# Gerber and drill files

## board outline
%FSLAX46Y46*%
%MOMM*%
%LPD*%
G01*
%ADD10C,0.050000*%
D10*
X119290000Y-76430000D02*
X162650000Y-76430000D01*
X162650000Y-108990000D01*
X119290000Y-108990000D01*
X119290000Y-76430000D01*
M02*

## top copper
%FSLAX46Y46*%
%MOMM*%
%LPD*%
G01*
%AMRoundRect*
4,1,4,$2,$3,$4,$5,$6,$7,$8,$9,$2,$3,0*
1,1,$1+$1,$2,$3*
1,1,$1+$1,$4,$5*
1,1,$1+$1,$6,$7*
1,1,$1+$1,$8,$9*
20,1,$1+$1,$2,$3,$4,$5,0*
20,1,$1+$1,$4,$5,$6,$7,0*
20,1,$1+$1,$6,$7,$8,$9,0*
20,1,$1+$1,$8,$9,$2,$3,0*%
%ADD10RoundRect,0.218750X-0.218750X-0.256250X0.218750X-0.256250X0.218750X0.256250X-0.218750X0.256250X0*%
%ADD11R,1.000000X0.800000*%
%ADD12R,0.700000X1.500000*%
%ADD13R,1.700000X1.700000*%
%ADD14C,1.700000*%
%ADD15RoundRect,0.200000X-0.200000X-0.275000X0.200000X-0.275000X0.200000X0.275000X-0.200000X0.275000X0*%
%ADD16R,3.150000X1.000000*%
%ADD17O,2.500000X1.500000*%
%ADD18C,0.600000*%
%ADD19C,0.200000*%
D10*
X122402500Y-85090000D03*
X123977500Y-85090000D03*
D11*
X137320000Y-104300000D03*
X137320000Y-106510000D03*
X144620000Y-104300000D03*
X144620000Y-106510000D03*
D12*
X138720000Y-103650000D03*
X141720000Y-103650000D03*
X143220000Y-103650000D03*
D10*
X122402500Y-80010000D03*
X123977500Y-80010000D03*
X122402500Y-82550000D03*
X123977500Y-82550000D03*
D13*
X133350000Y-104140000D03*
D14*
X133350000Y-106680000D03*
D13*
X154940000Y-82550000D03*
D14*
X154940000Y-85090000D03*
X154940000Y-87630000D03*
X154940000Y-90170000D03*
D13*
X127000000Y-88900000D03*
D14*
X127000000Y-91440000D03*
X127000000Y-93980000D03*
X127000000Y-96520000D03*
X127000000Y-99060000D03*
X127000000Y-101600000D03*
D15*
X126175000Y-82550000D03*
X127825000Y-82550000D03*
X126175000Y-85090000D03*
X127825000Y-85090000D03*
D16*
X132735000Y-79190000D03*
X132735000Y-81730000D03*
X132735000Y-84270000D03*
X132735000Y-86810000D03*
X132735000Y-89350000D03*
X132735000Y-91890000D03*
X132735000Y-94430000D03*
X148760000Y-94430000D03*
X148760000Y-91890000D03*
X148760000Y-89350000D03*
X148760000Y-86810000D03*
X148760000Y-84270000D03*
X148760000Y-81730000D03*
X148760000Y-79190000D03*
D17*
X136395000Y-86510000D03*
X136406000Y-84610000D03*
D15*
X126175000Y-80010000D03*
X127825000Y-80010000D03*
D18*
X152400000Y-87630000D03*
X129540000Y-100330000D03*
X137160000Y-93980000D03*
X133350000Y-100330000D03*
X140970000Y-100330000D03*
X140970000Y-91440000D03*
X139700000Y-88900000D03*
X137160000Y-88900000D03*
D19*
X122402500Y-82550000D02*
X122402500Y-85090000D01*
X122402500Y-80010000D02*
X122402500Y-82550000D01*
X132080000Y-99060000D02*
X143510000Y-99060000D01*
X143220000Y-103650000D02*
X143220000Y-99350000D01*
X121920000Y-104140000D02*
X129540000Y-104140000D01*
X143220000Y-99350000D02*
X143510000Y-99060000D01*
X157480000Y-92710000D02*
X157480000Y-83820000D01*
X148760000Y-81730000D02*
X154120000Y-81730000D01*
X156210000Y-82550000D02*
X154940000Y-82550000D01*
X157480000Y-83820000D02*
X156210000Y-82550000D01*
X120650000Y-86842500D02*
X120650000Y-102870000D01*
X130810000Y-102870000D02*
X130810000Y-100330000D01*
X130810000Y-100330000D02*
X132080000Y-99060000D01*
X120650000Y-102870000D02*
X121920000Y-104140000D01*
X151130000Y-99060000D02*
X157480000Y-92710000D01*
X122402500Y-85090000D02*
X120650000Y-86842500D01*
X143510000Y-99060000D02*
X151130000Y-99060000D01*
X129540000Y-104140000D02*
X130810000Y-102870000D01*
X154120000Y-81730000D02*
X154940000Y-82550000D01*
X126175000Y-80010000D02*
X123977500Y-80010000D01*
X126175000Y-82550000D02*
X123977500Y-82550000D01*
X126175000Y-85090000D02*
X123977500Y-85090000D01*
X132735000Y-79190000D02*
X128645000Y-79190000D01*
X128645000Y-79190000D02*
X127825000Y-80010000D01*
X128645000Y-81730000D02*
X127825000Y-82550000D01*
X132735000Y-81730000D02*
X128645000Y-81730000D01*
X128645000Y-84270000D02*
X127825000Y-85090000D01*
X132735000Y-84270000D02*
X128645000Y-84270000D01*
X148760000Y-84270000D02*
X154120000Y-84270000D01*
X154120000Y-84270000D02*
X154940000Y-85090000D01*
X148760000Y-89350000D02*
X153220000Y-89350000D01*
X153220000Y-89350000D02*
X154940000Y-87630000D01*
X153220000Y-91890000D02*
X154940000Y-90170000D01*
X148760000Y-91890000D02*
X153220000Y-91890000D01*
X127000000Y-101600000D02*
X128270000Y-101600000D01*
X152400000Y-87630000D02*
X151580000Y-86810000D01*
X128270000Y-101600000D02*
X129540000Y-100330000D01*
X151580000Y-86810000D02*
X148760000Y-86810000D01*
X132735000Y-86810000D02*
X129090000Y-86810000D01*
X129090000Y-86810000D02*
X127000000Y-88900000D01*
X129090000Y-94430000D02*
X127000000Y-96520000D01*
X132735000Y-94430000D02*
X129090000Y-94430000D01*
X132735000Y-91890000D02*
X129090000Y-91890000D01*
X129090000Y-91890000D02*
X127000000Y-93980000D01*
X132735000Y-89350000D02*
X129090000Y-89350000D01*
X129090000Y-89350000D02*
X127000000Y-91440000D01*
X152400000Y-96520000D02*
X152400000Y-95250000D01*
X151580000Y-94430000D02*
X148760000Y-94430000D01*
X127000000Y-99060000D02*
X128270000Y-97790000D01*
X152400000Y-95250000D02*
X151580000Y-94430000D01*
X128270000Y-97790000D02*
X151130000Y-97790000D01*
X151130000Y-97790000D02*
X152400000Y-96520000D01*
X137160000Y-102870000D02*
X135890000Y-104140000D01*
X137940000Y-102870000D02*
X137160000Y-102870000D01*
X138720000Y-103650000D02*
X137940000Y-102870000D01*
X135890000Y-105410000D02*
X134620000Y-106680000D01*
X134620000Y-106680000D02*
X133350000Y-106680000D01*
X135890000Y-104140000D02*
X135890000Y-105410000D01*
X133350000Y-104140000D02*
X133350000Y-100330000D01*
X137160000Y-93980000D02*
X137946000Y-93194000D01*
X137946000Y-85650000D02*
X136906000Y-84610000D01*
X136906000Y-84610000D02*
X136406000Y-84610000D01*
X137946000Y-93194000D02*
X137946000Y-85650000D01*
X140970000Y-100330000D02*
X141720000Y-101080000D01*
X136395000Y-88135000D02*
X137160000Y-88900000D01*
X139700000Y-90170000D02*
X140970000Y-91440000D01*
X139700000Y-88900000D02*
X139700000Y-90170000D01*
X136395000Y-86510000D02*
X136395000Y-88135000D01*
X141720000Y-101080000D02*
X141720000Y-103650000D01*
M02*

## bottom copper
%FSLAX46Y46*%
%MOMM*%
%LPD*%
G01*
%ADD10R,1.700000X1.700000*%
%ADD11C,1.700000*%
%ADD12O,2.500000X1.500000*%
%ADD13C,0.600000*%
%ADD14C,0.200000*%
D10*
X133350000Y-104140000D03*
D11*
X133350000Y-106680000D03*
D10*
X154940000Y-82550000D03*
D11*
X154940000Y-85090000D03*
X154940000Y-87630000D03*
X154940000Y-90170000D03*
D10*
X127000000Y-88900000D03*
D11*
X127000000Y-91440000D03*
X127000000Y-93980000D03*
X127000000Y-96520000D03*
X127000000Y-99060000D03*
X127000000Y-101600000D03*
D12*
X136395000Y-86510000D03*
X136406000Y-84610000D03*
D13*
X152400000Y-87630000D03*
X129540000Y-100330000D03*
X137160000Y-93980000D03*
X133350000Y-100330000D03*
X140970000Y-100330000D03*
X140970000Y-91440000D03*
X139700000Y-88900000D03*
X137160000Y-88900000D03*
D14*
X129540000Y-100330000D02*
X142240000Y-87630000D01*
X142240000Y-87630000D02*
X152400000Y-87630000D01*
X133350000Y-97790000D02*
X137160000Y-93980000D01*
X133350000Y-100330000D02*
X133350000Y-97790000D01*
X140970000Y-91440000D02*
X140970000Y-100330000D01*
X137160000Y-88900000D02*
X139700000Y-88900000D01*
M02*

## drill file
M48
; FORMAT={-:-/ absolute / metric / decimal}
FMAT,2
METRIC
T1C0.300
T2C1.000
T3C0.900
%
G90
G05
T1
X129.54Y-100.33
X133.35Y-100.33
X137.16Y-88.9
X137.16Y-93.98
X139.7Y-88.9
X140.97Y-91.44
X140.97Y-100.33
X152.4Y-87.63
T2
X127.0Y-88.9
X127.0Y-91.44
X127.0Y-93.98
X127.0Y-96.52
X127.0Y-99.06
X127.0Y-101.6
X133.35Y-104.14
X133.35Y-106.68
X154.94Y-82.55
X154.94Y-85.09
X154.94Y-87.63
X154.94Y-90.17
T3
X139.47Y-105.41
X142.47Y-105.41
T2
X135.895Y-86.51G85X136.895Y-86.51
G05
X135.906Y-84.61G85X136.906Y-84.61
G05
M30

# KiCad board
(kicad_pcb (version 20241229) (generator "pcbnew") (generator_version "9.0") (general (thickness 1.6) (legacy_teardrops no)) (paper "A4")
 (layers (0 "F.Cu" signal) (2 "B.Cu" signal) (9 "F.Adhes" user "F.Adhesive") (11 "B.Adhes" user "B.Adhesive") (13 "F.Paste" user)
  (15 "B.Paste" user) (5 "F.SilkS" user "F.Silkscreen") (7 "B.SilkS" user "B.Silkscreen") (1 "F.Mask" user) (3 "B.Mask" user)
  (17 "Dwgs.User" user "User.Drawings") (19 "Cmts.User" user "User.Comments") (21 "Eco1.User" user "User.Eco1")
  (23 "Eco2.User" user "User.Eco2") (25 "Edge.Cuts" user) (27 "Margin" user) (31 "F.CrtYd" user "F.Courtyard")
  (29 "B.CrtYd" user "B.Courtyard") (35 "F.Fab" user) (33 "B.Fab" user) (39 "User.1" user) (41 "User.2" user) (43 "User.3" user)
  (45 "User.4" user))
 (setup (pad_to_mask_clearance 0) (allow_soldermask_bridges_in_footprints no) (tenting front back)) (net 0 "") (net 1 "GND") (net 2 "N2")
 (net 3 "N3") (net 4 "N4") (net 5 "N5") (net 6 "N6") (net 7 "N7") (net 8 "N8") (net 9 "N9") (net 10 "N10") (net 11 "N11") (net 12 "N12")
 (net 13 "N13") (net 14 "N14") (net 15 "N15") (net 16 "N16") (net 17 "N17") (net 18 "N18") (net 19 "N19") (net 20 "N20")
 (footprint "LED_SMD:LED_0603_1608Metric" (layer "F.Cu") (at 123.19 85.09)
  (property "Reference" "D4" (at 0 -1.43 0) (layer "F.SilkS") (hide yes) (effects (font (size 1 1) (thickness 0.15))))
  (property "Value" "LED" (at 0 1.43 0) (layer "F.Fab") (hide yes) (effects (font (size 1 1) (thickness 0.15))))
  (pad "1" smd roundrect (at -0.7875 0) (size 0.875 0.95) (layers "F.Cu" "F.Mask" "F.Paste") (roundrect_rratio 0.25) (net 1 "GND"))
  (pad "2" smd roundrect (at 0.7875 0) (size 0.875 0.95) (layers "F.Cu" "F.Mask" "F.Paste") (roundrect_rratio 0.25) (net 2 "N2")))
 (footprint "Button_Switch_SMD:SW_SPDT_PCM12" (layer "F.Cu") (at 140.97 105.08)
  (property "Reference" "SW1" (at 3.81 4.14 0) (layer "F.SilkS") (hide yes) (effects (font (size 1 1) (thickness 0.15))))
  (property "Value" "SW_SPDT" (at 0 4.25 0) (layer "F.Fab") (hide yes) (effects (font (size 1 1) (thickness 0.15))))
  (pad "" smd rect (at -3.65 -0.78) (size 1 0.8) (layers "F.Cu" "F.Mask" "F.Paste"))
  (pad "" smd rect (at -3.65 1.43) (size 1 0.8) (layers "F.Cu" "F.Mask" "F.Paste"))
  (pad "" np_thru_hole circle (at -1.5 0.33) (size 0.9 0.9) (drill 0.9) (layers "*.Cu" "*.Mask"))
  (pad "" np_thru_hole circle (at 1.5 0.33) (size 0.9 0.9) (drill 0.9) (layers "*.Cu" "*.Mask"))
  (pad "" smd rect (at 3.65 -0.78) (size 1 0.8) (layers "F.Cu" "F.Mask" "F.Paste"))
  (pad "" smd rect (at 3.65 1.43) (size 1 0.8) (layers "F.Cu" "F.Mask" "F.Paste"))
  (pad "1" smd rect (at -2.25 -1.43) (size 0.7 1.5) (layers "F.Cu" "F.Mask" "F.Paste") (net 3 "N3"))
  (pad "2" smd rect (at 0.75 -1.43) (size 0.7 1.5) (layers "F.Cu" "F.Mask" "F.Paste") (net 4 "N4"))
  (pad "3" smd rect (at 2.25 -1.43) (size 0.7 1.5) (layers "F.Cu" "F.Mask" "F.Paste") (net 1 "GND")))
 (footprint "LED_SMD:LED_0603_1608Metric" (layer "F.Cu") (at 123.19 80.01)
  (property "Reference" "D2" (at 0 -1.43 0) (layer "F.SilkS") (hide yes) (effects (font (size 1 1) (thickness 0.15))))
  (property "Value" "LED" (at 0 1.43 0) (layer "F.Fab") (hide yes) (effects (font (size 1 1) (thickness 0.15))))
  (pad "1" smd roundrect (at -0.7875 0) (size 0.875 0.95) (layers "F.Cu" "F.Mask" "F.Paste") (roundrect_rratio 0.25) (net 1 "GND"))
  (pad "2" smd roundrect (at 0.7875 0) (size 0.875 0.95) (layers "F.Cu" "F.Mask" "F.Paste") (roundrect_rratio 0.25) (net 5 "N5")))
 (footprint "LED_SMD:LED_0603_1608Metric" (layer "F.Cu") (at 123.19 82.55)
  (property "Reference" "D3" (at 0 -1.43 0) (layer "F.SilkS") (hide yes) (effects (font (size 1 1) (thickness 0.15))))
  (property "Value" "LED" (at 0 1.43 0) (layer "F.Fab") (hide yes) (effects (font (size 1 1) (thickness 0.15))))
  (pad "1" smd roundrect (at -0.7875 0) (size 0.875 0.95) (layers "F.Cu" "F.Mask" "F.Paste") (roundrect_rratio 0.25) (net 1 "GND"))
  (pad "2" smd roundrect (at 0.7875 0) (size 0.875 0.95) (layers "F.Cu" "F.Mask" "F.Paste") (roundrect_rratio 0.25) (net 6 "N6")))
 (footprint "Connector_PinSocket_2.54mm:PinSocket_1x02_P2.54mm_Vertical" (layer "F.Cu") (at 133.35 104.14)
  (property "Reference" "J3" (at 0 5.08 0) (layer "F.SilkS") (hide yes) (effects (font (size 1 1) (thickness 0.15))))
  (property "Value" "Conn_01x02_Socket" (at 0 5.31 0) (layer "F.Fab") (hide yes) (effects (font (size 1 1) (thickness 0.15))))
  (pad "1" thru_hole rect (at 0 0) (size 1.7 1.7) (drill 1) (layers "*.Cu" "*.Mask") (remove_unused_layers no) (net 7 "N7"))
  (pad "2" thru_hole circle (at 0 2.54) (size 1.7 1.7) (drill 1) (layers "*.Cu" "*.Mask") (remove_unused_layers no) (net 3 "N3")))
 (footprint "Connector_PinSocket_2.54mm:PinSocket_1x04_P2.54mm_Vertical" (layer "F.Cu") (at 154.94 82.55)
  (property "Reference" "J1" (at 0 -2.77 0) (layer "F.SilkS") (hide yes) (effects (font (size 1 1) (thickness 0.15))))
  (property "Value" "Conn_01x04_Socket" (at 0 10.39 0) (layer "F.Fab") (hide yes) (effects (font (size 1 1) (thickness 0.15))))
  (pad "1" thru_hole rect (at 0 0) (size 1.7 1.7) (drill 1) (layers "*.Cu" "*.Mask") (remove_unused_layers no) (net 1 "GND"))
  (pad "2" thru_hole circle (at 0 2.54) (size 1.7 1.7) (drill 1) (layers "*.Cu" "*.Mask") (remove_unused_layers no) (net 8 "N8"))
  (pad "3" thru_hole circle (at 0 5.08) (size 1.7 1.7) (drill 1) (layers "*.Cu" "*.Mask") (remove_unused_layers no) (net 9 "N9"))
  (pad "4" thru_hole circle (at 0 7.62) (size 1.7 1.7) (drill 1) (layers "*.Cu" "*.Mask") (remove_unused_layers no) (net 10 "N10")))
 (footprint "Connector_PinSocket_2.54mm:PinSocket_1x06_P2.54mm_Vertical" (layer "F.Cu") (at 127 88.9)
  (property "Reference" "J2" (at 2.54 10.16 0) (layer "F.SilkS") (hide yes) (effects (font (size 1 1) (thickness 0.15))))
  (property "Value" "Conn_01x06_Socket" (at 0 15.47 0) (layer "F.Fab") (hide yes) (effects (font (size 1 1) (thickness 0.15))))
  (pad "1" thru_hole rect (at 0 0) (size 1.7 1.7) (drill 1) (layers "*.Cu" "*.Mask") (remove_unused_layers no) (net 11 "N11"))
  (pad "2" thru_hole circle (at 0 2.54) (size 1.7 1.7) (drill 1) (layers "*.Cu" "*.Mask") (remove_unused_layers no) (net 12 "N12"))
  (pad "3" thru_hole circle (at 0 5.08) (size 1.7 1.7) (drill 1) (layers "*.Cu" "*.Mask") (remove_unused_layers no) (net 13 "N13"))
  (pad "4" thru_hole circle (at 0 7.62) (size 1.7 1.7) (drill 1) (layers "*.Cu" "*.Mask") (remove_unused_layers no) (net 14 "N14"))
  (pad "5" thru_hole circle (at 0 10.16) (size 1.7 1.7) (drill 1) (layers "*.Cu" "*.Mask") (remove_unused_layers no) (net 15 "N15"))
  (pad "6" thru_hole circle (at 0 12.7) (size 1.7 1.7) (drill 1) (layers "*.Cu" "*.Mask") (remove_unused_layers no) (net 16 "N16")))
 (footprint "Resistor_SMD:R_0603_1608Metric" (layer "F.Cu") (at 127 82.55)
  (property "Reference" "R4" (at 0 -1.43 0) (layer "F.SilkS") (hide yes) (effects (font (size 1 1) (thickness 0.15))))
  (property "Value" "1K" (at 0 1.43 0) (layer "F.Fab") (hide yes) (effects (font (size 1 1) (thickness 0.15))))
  (pad "1" smd roundrect (at -0.825 0) (size 0.8 0.95) (layers "F.Cu" "F.Mask" "F.Paste") (roundrect_rratio 0.25) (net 6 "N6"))
  (pad "2" smd roundrect (at 0.825 0) (size 0.8 0.95) (layers "F.Cu" "F.Mask" "F.Paste") (roundrect_rratio 0.25) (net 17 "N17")))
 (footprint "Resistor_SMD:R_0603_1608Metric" (layer "F.Cu") (at 127 85.09)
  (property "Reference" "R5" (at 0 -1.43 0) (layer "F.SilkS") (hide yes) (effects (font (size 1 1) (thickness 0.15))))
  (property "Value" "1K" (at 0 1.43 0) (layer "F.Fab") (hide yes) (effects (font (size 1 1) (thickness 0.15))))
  (pad "1" smd roundrect (at -0.825 0) (size 0.8 0.95) (layers "F.Cu" "F.Mask" "F.Paste") (roundrect_rratio 0.25) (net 2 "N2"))
  (pad "2" smd roundrect (at 0.825 0) (size 0.8 0.95) (layers "F.Cu" "F.Mask" "F.Paste") (roundrect_rratio 0.25) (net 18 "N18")))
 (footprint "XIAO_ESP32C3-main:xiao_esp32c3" (layer "F.Cu") (at 141.335 88.61)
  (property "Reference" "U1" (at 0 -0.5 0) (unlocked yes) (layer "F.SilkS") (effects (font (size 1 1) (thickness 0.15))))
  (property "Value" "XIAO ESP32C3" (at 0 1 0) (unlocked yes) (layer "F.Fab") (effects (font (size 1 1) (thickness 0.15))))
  (pad "1" smd rect (at -8.6 -9.42) (size 3.15 1) (layers "F.Cu" "F.Mask" "F.Paste") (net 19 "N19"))
  (pad "2" smd rect (at -8.6 -6.88) (size 3.15 1) (layers "F.Cu" "F.Mask" "F.Paste") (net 17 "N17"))
  (pad "3" smd rect (at -8.6 -4.34) (size 3.15 1) (layers "F.Cu" "F.Mask" "F.Paste") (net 18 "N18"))
  (pad "4" smd rect (at -8.6 -1.8) (size 3.15 1) (layers "F.Cu" "F.Mask" "F.Paste") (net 11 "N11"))
  (pad "5" smd rect (at -8.6 0.74) (size 3.15 1) (layers "F.Cu" "F.Mask" "F.Paste") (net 12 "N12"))
  (pad "6" smd rect (at -8.6 3.28) (size 3.15 1) (layers "F.Cu" "F.Mask" "F.Paste") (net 13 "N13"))
  (pad "7" smd rect (at -8.6 5.82) (size 3.15 1) (layers "F.Cu" "F.Mask" "F.Paste") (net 14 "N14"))
  (pad "8" smd rect (at 7.425 5.82) (size 3.15 1) (layers "F.Cu" "F.Mask" "F.Paste") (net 15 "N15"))
  (pad "9" smd rect (at 7.425 3.28) (size 3.15 1) (layers "F.Cu" "F.Mask" "F.Paste") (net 10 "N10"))
  (pad "10" smd rect (at 7.425 0.74) (size 3.15 1) (layers "F.Cu" "F.Mask" "F.Paste") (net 9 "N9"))
  (pad "11" smd rect (at 7.425 -1.8) (size 3.15 1) (layers "F.Cu" "F.Mask" "F.Paste") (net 16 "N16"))
  (pad "12" smd rect (at 7.425 -4.34) (size 3.15 1) (layers "F.Cu" "F.Mask" "F.Paste") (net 8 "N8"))
  (pad "13" smd rect (at 7.425 -6.88) (size 3.15 1) (layers "F.Cu" "F.Mask" "F.Paste") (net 1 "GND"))
  (pad "14" smd rect (at 7.425 -9.42) (size 3.15 1) (layers "F.Cu" "F.Mask" "F.Paste") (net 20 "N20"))
  (pad "B+" thru_hole oval (at -4.94 -2.1) (size 2.5 1.5) (drill oval 2 1) (layers "*.Cu" "*.Mask") (remove_unused_layers no) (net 4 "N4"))
  (pad "B-" thru_hole oval (at -4.929 -4) (size 2.5 1.5) (drill oval 2 1) (layers "*.Cu" "*.Mask") (remove_unused_layers no) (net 7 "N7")))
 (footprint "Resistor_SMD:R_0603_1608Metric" (layer "F.Cu") (at 127 80.01)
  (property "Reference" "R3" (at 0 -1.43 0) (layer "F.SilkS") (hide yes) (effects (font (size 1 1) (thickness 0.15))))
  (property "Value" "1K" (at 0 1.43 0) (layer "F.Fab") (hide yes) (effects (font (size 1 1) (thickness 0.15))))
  (pad "1" smd roundrect (at -0.825 0) (size 0.8 0.95) (layers "F.Cu" "F.Mask" "F.Paste") (roundrect_rratio 0.25) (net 5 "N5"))
  (pad "2" smd roundrect (at 0.825 0) (size 0.8 0.95) (layers "F.Cu" "F.Mask" "F.Paste") (roundrect_rratio 0.25) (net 19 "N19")))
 (gr_rect (start 119.29 76.43) (end 162.65 108.99) (stroke (width 0.05) (type default)) (fill no) (layer "Edge.Cuts"))
 (segment (start 122.4025 82.55) (end 122.4025 85.09) (width 0.2) (layer "F.Cu") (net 1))
 (segment (start 122.4025 80.01) (end 122.4025 82.55) (width 0.2) (layer "F.Cu") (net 1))
 (segment (start 132.08 99.06) (end 143.51 99.06) (width 0.2) (layer "F.Cu") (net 1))
 (segment (start 143.22 103.65) (end 143.22 99.35) (width 0.2) (layer "F.Cu") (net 1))
 (segment (start 121.92 104.14) (end 129.54 104.14) (width 0.2) (layer "F.Cu") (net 1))
 (segment (start 143.22 99.35) (end 143.51 99.06) (width 0.2) (layer "F.Cu") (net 1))
 (segment (start 157.48 92.71) (end 157.48 83.82) (width 0.2) (layer "F.Cu") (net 1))
 (segment (start 148.76 81.73) (end 154.12 81.73) (width 0.2) (layer "F.Cu") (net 1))
 (segment (start 156.21 82.55) (end 154.94 82.55) (width 0.2) (layer "F.Cu") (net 1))
 (segment (start 157.48 83.82) (end 156.21 82.55) (width 0.2) (layer "F.Cu") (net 1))
 (segment (start 120.65 86.8425) (end 120.65 102.87) (width 0.2) (layer "F.Cu") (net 1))
 (segment (start 130.81 102.87) (end 130.81 100.33) (width 0.2) (layer "F.Cu") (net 1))
 (segment (start 130.81 100.33) (end 132.08 99.06) (width 0.2) (layer "F.Cu") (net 1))
 (segment (start 120.65 102.87) (end 121.92 104.14) (width 0.2) (layer "F.Cu") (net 1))
 (segment (start 151.13 99.06) (end 157.48 92.71) (width 0.2) (layer "F.Cu") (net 1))
 (segment (start 122.4025 85.09) (end 120.65 86.8425) (width 0.2) (layer "F.Cu") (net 1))
 (segment (start 143.51 99.06) (end 151.13 99.06) (width 0.2) (layer "F.Cu") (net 1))
 (segment (start 129.54 104.14) (end 130.81 102.87) (width 0.2) (layer "F.Cu") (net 1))
 (segment (start 154.12 81.73) (end 154.94 82.55) (width 0.2) (layer "F.Cu") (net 1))
 (segment (start 126.175 80.01) (end 123.9775 80.01) (width 0.2) (layer "F.Cu") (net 5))
 (segment (start 126.175 82.55) (end 123.9775 82.55) (width 0.2) (layer "F.Cu") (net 6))
 (segment (start 126.175 85.09) (end 123.9775 85.09) (width 0.2) (layer "F.Cu") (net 2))
 (segment (start 132.735 79.19) (end 128.645 79.19) (width 0.2) (layer "F.Cu") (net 19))
 (segment (start 128.645 79.19) (end 127.825 80.01) (width 0.2) (layer "F.Cu") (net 19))
 (segment (start 128.645 81.73) (end 127.825 82.55) (width 0.2) (layer "F.Cu") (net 17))
 (segment (start 132.735 81.73) (end 128.645 81.73) (width 0.2) (layer "F.Cu") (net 17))
 (segment (start 128.645 84.27) (end 127.825 85.09) (width 0.2) (layer "F.Cu") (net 18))
 (segment (start 132.735 84.27) (end 128.645 84.27) (width 0.2) (layer "F.Cu") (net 18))
 (segment (start 148.76 84.27) (end 154.12 84.27) (width 0.2) (layer "F.Cu") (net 8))
 (segment (start 154.12 84.27) (end 154.94 85.09) (width 0.2) (layer "F.Cu") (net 8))
 (segment (start 148.76 89.35) (end 153.22 89.35) (width 0.2) (layer "F.Cu") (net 9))
 (segment (start 153.22 89.35) (end 154.94 87.63) (width 0.2) (layer "F.Cu") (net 9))
 (segment (start 153.22 91.89) (end 154.94 90.17) (width 0.2) (layer "F.Cu") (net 10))
 (segment (start 148.76 91.89) (end 153.22 91.89) (width 0.2) (layer "F.Cu") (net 10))
 (segment (start 127 101.6) (end 128.27 101.6) (width 0.2) (layer "F.Cu") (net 16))
 (segment (start 152.4 87.63) (end 151.58 86.81) (width 0.2) (layer "F.Cu") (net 16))
 (segment (start 128.27 101.6) (end 129.54 100.33) (width 0.2) (layer "F.Cu") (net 16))
 (segment (start 151.58 86.81) (end 148.76 86.81) (width 0.2) (layer "F.Cu") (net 16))
 (via (at 152.4 87.63) (size 0.6) (drill 0.3) (layers "F.Cu" "B.Cu") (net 16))
 (via (at 129.54 100.33) (size 0.6) (drill 0.3) (layers "F.Cu" "B.Cu") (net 16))
 (segment (start 129.54 100.33) (end 142.24 87.63) (width 0.2) (layer "B.Cu") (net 16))
 (segment (start 142.24 87.63) (end 152.4 87.63) (width 0.2) (layer "B.Cu") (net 16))
 (segment (start 132.735 86.81) (end 129.09 86.81) (width 0.2) (layer "F.Cu") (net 11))
 (segment (start 129.09 86.81) (end 127 88.9) (width 0.2) (layer "F.Cu") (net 11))
 (segment (start 129.09 94.43) (end 127 96.52) (width 0.2) (layer "F.Cu") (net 14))
 (segment (start 132.735 94.43) (end 129.09 94.43) (width 0.2) (layer "F.Cu") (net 14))
 (segment (start 132.735 91.89) (end 129.09 91.89) (width 0.2) (layer "F.Cu") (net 13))
 (segment (start 129.09 91.89) (end 127 93.98) (width 0.2) (layer "F.Cu") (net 13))
 (segment (start 132.735 89.35) (end 129.09 89.35) (width 0.2) (layer "F.Cu") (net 12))
 (segment (start 129.09 89.35) (end 127 91.44) (width 0.2) (layer "F.Cu") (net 12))
 (segment (start 152.4 96.52) (end 152.4 95.25) (width 0.2) (layer "F.Cu") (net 15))
 (segment (start 151.58 94.43) (end 148.76 94.43) (width 0.2) (layer "F.Cu") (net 15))
 (segment (start 127 99.06) (end 128.27 97.79) (width 0.2) (layer "F.Cu") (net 15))
 (segment (start 152.4 95.25) (end 151.58 94.43) (width 0.2) (layer "F.Cu") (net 15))
 (segment (start 128.27 97.79) (end 151.13 97.79) (width 0.2) (layer "F.Cu") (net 15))
 (segment (start 151.13 97.79) (end 152.4 96.52) (width 0.2) (layer "F.Cu") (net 15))
 (segment (start 137.16 102.87) (end 135.89 104.14) (width 0.2) (layer "F.Cu") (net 3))
 (segment (start 137.94 102.87) (end 137.16 102.87) (width 0.2) (layer "F.Cu") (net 3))
 (segment (start 138.72 103.65) (end 137.94 102.87) (width 0.2) (layer "F.Cu") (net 3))
 (segment (start 135.89 105.41) (end 134.62 106.68) (width 0.2) (layer "F.Cu") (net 3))
 (segment (start 134.62 106.68) (end 133.35 106.68) (width 0.2) (layer "F.Cu") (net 3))
 (segment (start 135.89 104.14) (end 135.89 105.41) (width 0.2) (layer "F.Cu") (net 3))
 (segment (start 133.35 104.14) (end 133.35 100.33) (width 0.2) (layer "F.Cu") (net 7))
 (segment (start 137.16 93.98) (end 137.946 93.194) (width 0.2) (layer "F.Cu") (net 7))
 (segment (start 137.946 85.65) (end 136.906 84.61) (width 0.2) (layer "F.Cu") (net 7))
 (segment (start 136.906 84.61) (end 136.406 84.61) (width 0.2) (layer "F.Cu") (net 7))
 (segment (start 137.946 93.194) (end 137.946 85.65) (width 0.2) (layer "F.Cu") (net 7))
 (via (at 137.16 93.98) (size 0.6) (drill 0.3) (layers "F.Cu" "B.Cu") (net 7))
 (via (at 133.35 100.33) (size 0.6) (drill 0.3) (layers "F.Cu" "B.Cu") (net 7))
 (segment (start 133.35 97.79) (end 137.16 93.98) (width 0.2) (layer "B.Cu") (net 7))
 (segment (start 133.35 100.33) (end 133.35 97.79) (width 0.2) (layer "B.Cu") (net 7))
 (segment (start 140.97 100.33) (end 141.72 101.08) (width 0.2) (layer "F.Cu") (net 4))
 (segment (start 136.395 88.135) (end 137.16 88.9) (width 0.2) (layer "F.Cu") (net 4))
 (segment (start 139.7 90.17) (end 140.97 91.44) (width 0.2) (layer "F.Cu") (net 4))
 (segment (start 139.7 88.9) (end 139.7 90.17) (width 0.2) (layer "F.Cu") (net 4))
 (segment (start 136.395 86.51) (end 136.395 88.135) (width 0.2) (layer "F.Cu") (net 4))
 (segment (start 141.72 101.08) (end 141.72 103.65) (width 0.2) (layer "F.Cu") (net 4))
 (via (at 140.97 100.33) (size 0.6) (drill 0.3) (layers "F.Cu" "B.Cu") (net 4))
 (via (at 140.97 91.44) (size 0.6) (drill 0.3) (layers "F.Cu" "B.Cu") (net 4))
 (via (at 139.7 88.9) (size 0.6) (drill 0.3) (layers "F.Cu" "B.Cu") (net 4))
 (via (at 137.16 88.9) (size 0.6) (drill 0.3) (layers "F.Cu" "B.Cu") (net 4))
 (segment (start 140.97 91.44) (end 140.97 100.33) (width 0.2) (layer "B.Cu") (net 4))
 (segment (start 137.16 88.9) (end 139.7 88.9) (width 0.2) (layer "B.Cu") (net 4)))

